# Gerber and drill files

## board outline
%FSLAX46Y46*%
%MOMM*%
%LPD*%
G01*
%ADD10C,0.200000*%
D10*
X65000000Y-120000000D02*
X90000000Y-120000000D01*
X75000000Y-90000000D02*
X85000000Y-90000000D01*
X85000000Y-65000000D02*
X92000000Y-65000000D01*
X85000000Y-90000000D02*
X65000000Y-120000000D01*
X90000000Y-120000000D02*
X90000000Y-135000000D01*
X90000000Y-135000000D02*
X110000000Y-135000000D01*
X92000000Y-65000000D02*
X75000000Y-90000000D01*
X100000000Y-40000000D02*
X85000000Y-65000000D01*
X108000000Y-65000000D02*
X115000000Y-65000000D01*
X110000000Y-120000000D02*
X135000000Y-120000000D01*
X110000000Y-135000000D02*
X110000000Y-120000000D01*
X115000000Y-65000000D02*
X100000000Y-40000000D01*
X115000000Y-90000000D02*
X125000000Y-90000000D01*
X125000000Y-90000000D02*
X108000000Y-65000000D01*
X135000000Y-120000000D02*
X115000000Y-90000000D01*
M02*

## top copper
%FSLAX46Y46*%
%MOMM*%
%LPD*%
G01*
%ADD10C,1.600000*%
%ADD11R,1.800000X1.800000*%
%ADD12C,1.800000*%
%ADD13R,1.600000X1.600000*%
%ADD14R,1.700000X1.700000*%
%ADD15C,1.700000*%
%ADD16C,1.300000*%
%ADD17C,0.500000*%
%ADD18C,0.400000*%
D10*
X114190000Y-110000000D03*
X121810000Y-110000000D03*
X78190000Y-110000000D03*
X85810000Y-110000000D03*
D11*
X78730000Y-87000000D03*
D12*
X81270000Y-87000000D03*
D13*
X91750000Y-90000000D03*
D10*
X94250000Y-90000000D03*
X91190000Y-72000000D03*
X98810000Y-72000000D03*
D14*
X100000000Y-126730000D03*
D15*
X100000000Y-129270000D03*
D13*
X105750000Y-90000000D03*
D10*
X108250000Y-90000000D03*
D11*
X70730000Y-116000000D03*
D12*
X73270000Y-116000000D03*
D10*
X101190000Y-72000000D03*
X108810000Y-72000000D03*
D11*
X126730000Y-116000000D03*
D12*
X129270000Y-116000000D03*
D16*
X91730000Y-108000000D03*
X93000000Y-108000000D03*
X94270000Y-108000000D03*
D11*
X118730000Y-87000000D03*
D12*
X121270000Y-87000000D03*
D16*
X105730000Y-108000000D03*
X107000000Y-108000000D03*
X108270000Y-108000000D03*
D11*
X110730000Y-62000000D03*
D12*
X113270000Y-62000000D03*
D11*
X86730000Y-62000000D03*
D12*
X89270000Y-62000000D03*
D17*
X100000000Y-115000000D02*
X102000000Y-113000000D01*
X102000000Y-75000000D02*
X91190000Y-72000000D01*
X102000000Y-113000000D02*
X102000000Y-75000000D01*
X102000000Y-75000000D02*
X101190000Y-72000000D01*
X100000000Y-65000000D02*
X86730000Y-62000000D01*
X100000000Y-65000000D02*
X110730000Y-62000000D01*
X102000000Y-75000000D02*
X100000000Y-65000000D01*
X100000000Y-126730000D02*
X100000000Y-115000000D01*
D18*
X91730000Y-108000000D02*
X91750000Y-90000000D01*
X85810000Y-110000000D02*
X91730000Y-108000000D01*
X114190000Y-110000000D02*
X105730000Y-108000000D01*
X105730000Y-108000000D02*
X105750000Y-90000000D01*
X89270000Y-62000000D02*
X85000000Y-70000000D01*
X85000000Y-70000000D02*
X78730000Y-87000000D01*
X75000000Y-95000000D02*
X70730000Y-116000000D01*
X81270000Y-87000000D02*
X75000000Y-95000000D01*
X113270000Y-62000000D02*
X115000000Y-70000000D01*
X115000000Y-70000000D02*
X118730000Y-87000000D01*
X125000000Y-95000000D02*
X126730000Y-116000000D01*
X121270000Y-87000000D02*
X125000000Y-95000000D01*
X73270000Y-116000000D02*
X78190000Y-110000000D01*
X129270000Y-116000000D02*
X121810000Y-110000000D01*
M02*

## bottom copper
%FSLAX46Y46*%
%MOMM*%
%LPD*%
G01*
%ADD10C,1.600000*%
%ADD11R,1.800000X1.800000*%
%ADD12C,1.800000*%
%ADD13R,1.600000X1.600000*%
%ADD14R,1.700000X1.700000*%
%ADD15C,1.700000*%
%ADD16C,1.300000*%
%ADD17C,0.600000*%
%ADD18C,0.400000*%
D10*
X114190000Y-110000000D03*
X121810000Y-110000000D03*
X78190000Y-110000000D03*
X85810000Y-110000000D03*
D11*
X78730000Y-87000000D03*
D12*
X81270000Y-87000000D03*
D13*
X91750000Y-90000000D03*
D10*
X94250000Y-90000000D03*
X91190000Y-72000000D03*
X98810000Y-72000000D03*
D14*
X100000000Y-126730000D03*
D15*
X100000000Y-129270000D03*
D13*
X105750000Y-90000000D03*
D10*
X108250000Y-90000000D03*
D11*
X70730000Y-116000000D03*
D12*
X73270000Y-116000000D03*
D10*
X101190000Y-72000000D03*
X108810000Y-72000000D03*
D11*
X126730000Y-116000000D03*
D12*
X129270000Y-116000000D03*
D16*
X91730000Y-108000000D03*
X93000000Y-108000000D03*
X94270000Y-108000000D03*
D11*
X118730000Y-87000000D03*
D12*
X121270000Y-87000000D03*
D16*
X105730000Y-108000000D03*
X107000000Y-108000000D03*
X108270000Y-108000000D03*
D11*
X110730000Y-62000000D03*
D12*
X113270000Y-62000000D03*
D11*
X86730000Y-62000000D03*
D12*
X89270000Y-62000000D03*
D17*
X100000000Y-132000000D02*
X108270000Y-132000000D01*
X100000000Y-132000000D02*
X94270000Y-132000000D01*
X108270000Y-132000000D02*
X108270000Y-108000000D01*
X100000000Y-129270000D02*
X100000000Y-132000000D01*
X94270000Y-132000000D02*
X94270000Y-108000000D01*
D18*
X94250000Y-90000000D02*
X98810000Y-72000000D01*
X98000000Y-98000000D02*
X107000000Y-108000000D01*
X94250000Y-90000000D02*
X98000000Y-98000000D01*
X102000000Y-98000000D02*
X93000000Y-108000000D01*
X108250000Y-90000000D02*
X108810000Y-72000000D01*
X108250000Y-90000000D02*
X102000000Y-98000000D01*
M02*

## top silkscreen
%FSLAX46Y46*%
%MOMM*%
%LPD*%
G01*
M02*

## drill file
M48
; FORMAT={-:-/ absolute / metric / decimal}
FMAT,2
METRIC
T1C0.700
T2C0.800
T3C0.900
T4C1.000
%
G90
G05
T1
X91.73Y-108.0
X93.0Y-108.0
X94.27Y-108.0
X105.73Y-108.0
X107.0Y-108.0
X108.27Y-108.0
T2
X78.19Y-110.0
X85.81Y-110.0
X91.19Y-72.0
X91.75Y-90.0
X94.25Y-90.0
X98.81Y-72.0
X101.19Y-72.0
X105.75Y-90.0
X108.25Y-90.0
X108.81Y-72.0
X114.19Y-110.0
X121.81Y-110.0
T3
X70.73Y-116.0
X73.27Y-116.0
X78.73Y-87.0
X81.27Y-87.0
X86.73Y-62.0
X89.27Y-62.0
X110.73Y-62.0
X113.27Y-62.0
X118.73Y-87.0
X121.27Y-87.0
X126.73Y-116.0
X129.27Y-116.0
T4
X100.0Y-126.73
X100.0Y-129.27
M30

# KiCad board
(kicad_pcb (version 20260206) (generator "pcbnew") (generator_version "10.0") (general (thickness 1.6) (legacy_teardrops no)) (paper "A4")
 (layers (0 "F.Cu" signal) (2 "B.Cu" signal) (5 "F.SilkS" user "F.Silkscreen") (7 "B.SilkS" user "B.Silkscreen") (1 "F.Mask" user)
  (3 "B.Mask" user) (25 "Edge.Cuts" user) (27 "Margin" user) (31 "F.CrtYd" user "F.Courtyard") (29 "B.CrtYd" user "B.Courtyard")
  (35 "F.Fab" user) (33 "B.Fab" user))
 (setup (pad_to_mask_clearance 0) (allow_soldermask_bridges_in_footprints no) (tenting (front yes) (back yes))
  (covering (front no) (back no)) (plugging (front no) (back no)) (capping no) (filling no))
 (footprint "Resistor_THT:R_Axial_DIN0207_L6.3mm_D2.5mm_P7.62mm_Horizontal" (layer "F.Cu") (at 118 110)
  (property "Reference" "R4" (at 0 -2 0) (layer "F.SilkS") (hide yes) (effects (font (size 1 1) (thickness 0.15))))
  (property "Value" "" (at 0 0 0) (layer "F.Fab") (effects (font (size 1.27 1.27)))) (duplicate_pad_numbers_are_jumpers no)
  (pad "1" thru_hole circle (at -3.81 0) (size 1.6 1.6) (drill 0.8) (layers "*.Cu" "*.Mask") (remove_unused_layers no) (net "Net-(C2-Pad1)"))
  (pad "2" thru_hole circle (at 3.81 0) (size 1.6 1.6) (drill 0.8) (layers "*.Cu" "*.Mask") (remove_unused_layers no) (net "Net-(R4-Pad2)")))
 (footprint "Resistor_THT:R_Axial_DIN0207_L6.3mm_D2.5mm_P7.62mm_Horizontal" (layer "F.Cu") (at 82 110)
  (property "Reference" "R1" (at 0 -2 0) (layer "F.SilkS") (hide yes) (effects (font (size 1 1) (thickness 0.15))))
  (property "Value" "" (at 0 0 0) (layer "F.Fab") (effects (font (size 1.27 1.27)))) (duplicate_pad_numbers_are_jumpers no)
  (pad "1" thru_hole circle (at -3.81 0) (size 1.6 1.6) (drill 0.8) (layers "*.Cu" "*.Mask") (remove_unused_layers no) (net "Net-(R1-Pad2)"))
  (pad "2" thru_hole circle (at 3.81 0) (size 1.6 1.6) (drill 0.8) (layers "*.Cu" "*.Mask") (remove_unused_layers no) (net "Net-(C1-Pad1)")))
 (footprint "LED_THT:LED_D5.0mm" (layer "F.Cu") (at 80 87)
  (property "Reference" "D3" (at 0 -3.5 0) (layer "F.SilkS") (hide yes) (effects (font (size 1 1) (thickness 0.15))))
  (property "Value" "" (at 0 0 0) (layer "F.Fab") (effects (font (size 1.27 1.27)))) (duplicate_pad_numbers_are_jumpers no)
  (pad "1" thru_hole rect (at -1.27 0) (size 1.8 1.8) (drill 0.9) (layers "*.Cu" "*.Mask") (remove_unused_layers no) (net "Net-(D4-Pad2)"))
  (pad "2" thru_hole circle (at 1.27 0) (size 1.8 1.8) (drill 0.9) (layers "*.Cu" "*.Mask") (remove_unused_layers no) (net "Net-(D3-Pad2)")))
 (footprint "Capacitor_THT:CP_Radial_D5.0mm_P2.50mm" (layer "F.Cu") (at 93 90)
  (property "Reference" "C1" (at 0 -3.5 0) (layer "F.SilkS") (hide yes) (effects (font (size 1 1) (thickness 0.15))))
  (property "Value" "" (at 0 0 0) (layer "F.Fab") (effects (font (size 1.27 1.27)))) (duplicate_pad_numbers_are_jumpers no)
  (pad "1" thru_hole rect (at -1.25 0) (size 1.6 1.6) (drill 0.8) (layers "*.Cu" "*.Mask") (remove_unused_layers no) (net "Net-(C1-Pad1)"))
  (pad "2" thru_hole circle (at 1.25 0) (size 1.6 1.6) (drill 0.8) (layers "*.Cu" "*.Mask") (remove_unused_layers no) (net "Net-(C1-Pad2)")))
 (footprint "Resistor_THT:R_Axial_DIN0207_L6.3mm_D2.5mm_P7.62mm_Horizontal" (layer "F.Cu") (at 95 72)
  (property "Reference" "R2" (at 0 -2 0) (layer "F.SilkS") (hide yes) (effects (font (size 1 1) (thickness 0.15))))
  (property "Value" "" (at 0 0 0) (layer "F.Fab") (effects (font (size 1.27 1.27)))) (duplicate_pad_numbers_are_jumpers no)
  (pad "1" thru_hole circle (at -3.81 0) (size 1.6 1.6) (drill 0.8) (layers "*.Cu" "*.Mask") (remove_unused_layers no) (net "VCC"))
  (pad "2" thru_hole circle (at 3.81 0) (size 1.6 1.6) (drill 0.8) (layers "*.Cu" "*.Mask") (remove_unused_layers no) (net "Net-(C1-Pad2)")))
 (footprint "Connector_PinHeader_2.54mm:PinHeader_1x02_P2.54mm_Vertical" (layer "F.Cu") (at 100 128)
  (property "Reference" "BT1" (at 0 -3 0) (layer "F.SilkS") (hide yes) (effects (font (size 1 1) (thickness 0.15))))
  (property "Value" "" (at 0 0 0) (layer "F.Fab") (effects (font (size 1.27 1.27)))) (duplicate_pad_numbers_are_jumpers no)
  (pad "1" thru_hole rect (at 0 -1.27) (size 1.7 1.7) (drill 1) (layers "*.Cu" "*.Mask") (remove_unused_layers no) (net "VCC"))
  (pad "2" thru_hole circle (at 0 1.27) (size 1.7 1.7) (drill 1) (layers "*.Cu" "*.Mask") (remove_unused_layers no) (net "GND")))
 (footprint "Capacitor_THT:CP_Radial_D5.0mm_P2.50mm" (layer "F.Cu") (at 107 90)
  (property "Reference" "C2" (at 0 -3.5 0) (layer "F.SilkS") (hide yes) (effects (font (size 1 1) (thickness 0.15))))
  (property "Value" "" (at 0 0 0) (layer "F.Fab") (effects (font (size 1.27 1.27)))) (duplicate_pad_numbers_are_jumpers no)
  (pad "1" thru_hole rect (at -1.25 0) (size 1.6 1.6) (drill 0.8) (layers "*.Cu" "*.Mask") (remove_unused_layers no) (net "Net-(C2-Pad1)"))
  (pad "2" thru_hole circle (at 1.25 0) (size 1.6 1.6) (drill 0.8) (layers "*.Cu" "*.Mask") (remove_unused_layers no) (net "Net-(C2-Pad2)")))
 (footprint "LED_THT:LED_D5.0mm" (layer "F.Cu") (at 72 116)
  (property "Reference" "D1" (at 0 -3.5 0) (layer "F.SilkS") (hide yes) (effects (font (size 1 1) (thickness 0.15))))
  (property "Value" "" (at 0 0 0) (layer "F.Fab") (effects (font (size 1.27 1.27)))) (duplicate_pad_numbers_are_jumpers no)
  (pad "1" thru_hole rect (at -1.27 0) (size 1.8 1.8) (drill 0.9) (layers "*.Cu" "*.Mask") (remove_unused_layers no) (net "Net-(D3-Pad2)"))
  (pad "2" thru_hole circle (at 1.27 0) (size 1.8 1.8) (drill 0.9) (layers "*.Cu" "*.Mask") (remove_unused_layers no) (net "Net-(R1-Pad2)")))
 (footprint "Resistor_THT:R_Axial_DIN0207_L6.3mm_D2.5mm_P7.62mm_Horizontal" (layer "F.Cu") (at 105 72)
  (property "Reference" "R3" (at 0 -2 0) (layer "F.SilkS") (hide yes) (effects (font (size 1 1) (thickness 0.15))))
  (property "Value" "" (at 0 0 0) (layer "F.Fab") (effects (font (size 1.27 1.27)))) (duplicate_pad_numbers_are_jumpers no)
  (pad "1" thru_hole circle (at -3.81 0) (size 1.6 1.6) (drill 0.8) (layers "*.Cu" "*.Mask") (remove_unused_layers no) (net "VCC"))
  (pad "2" thru_hole circle (at 3.81 0) (size 1.6 1.6) (drill 0.8) (layers "*.Cu" "*.Mask") (remove_unused_layers no) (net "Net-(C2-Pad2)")))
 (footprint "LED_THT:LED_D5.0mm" (layer "F.Cu") (at 128 116)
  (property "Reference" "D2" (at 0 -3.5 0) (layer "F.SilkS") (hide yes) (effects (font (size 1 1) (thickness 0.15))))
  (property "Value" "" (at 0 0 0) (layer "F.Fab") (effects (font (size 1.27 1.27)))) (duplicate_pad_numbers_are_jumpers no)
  (pad "1" thru_hole rect (at -1.27 0) (size 1.8 1.8) (drill 0.9) (layers "*.Cu" "*.Mask") (remove_unused_layers no) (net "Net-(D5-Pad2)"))
  (pad "2" thru_hole circle (at 1.27 0) (size 1.8 1.8) (drill 0.9) (layers "*.Cu" "*.Mask") (remove_unused_layers no) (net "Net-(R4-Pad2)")))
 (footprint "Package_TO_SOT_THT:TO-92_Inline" (layer "F.Cu") (at 93 108)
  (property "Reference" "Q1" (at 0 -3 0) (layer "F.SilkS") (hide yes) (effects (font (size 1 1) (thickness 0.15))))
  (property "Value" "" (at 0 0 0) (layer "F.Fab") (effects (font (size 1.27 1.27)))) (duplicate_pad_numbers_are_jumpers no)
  (pad "1" thru_hole circle (at -1.27 0) (size 1.3 1.3) (drill 0.7) (layers "*.Cu" "*.Mask") (remove_unused_layers no) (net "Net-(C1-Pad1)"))
  (pad "2" thru_hole circle (at 0 0) (size 1.3 1.3) (drill 0.7) (layers "*.Cu" "*.Mask") (remove_unused_layers no) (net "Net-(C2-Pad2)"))
  (pad "3" thru_hole circle (at 1.27 0) (size 1.3 1.3) (drill 0.7) (layers "*.Cu" "*.Mask") (remove_unused_layers no) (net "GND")))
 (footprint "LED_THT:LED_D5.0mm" (layer "F.Cu") (at 120 87)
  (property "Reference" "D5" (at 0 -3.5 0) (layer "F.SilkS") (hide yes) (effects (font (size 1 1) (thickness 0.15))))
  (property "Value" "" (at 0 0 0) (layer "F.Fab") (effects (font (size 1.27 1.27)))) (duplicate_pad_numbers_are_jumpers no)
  (pad "1" thru_hole rect (at -1.27 0) (size 1.8 1.8) (drill 0.9) (layers "*.Cu" "*.Mask") (remove_unused_layers no) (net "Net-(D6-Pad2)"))
  (pad "2" thru_hole circle (at 1.27 0) (size 1.8 1.8) (drill 0.9) (layers "*.Cu" "*.Mask") (remove_unused_layers no) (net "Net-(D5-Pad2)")))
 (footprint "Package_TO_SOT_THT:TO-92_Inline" (layer "F.Cu") (at 107 108)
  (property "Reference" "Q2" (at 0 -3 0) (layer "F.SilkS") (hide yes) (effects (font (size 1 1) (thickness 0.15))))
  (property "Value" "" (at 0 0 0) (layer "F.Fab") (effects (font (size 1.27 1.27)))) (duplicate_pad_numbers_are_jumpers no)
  (pad "1" thru_hole circle (at -1.27 0) (size 1.3 1.3) (drill 0.7) (layers "*.Cu" "*.Mask") (remove_unused_layers no) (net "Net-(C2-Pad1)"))
  (pad "2" thru_hole circle (at 0 0) (size 1.3 1.3) (drill 0.7) (layers "*.Cu" "*.Mask") (remove_unused_layers no) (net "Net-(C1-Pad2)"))
  (pad "3" thru_hole circle (at 1.27 0) (size 1.3 1.3) (drill 0.7) (layers "*.Cu" "*.Mask") (remove_unused_layers no) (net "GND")))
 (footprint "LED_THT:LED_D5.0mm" (layer "F.Cu") (at 112 62)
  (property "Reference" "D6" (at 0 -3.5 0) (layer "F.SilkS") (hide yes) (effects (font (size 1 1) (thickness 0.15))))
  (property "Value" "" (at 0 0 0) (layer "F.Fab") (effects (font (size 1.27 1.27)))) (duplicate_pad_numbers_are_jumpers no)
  (pad "1" thru_hole rect (at -1.27 0) (size 1.8 1.8) (drill 0.9) (layers "*.Cu" "*.Mask") (remove_unused_layers no) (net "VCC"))
  (pad "2" thru_hole circle (at 1.27 0) (size 1.8 1.8) (drill 0.9) (layers "*.Cu" "*.Mask") (remove_unused_layers no) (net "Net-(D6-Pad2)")))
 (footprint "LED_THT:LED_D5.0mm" (layer "F.Cu") (at 88 62)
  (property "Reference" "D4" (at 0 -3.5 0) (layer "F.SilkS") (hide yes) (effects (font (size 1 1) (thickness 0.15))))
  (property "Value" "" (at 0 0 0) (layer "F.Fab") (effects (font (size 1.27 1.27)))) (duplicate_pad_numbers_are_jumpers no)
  (pad "1" thru_hole rect (at -1.27 0) (size 1.8 1.8) (drill 0.9) (layers "*.Cu" "*.Mask") (remove_unused_layers no) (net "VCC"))
  (pad "2" thru_hole circle (at 1.27 0) (size 1.8 1.8) (drill 0.9) (layers "*.Cu" "*.Mask") (remove_unused_layers no) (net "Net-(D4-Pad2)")))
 (gr_line (start 65 120) (end 90 120) (stroke (width 0.2) (type solid)) (layer "Edge.Cuts"))
 (gr_line (start 75 90) (end 85 90) (stroke (width 0.2) (type solid)) (layer "Edge.Cuts"))
 (gr_line (start 85 65) (end 92 65) (stroke (width 0.2) (type solid)) (layer "Edge.Cuts"))
 (gr_line (start 85 90) (end 65 120) (stroke (width 0.2) (type solid)) (layer "Edge.Cuts"))
 (gr_line (start 90 120) (end 90 135) (stroke (width 0.2) (type solid)) (layer "Edge.Cuts"))
 (gr_line (start 90 135) (end 110 135) (stroke (width 0.2) (type solid)) (layer "Edge.Cuts"))
 (gr_line (start 92 65) (end 75 90) (stroke (width 0.2) (type solid)) (layer "Edge.Cuts"))
 (gr_line (start 100 40) (end 85 65) (stroke (width 0.2) (type solid)) (layer "Edge.Cuts"))
 (gr_line (start 108 65) (end 115 65) (stroke (width 0.2) (type solid)) (layer "Edge.Cuts"))
 (gr_line (start 110 120) (end 135 120) (stroke (width 0.2) (type solid)) (layer "Edge.Cuts"))
 (gr_line (start 110 135) (end 110 120) (stroke (width 0.2) (type solid)) (layer "Edge.Cuts"))
 (gr_line (start 115 65) (end 100 40) (stroke (width 0.2) (type solid)) (layer "Edge.Cuts"))
 (gr_line (start 115 90) (end 125 90) (stroke (width 0.2) (type solid)) (layer "Edge.Cuts"))
 (gr_line (start 125 90) (end 108 65) (stroke (width 0.2) (type solid)) (layer "Edge.Cuts"))
 (gr_line (start 135 120) (end 115 90) (stroke (width 0.2) (type solid)) (layer "Edge.Cuts"))
 (segment (start 100 115) (end 102 113) (width 0.5) (layer "F.Cu") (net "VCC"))
 (segment (start 102 75) (end 91.19 72) (width 0.5) (layer "F.Cu") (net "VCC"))
 (segment (start 102 113) (end 102 75) (width 0.5) (layer "F.Cu") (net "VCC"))
 (segment (start 102 75) (end 101.19 72) (width 0.5) (layer "F.Cu") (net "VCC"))
 (segment (start 100 65) (end 86.73 62) (width 0.5) (layer "F.Cu") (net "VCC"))
 (segment (start 100 65) (end 110.73 62) (width 0.5) (layer "F.Cu") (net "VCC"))
 (segment (start 102 75) (end 100 65) (width 0.5) (layer "F.Cu") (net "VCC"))
 (segment (start 100 126.73) (end 100 115) (width 0.5) (layer "F.Cu") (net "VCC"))
 (segment (start 100 132) (end 108.27 132) (width 0.6) (layer "B.Cu") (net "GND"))
 (segment (start 100 132) (end 94.27 132) (width 0.6) (layer "B.Cu") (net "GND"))
 (segment (start 108.27 132) (end 108.27 108) (width 0.6) (layer "B.Cu") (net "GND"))
 (segment (start 100 129.27) (end 100 132) (width 0.6) (layer "B.Cu") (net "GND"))
 (segment (start 94.27 132) (end 94.27 108) (width 0.6) (layer "B.Cu") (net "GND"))
 (segment (start 91.73 108) (end 91.75 90) (width 0.4) (layer "F.Cu") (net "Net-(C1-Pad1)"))
 (segment (start 85.81 110) (end 91.73 108) (width 0.4) (layer "F.Cu") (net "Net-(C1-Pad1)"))
 (segment (start 114.19 110) (end 105.73 108) (width 0.4) (layer "F.Cu") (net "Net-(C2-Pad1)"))
 (segment (start 105.73 108) (end 105.75 90) (width 0.4) (layer "F.Cu") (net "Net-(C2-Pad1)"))
 (segment (start 94.25 90) (end 98.81 72) (width 0.4) (layer "B.Cu") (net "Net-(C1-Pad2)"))
 (segment (start 98 98) (end 107 108) (width 0.4) (layer "B.Cu") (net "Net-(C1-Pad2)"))
 (segment (start 94.25 90) (end 98 98) (width 0.4) (layer "B.Cu") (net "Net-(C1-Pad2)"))
 (segment (start 102 98) (end 93 108) (width 0.4) (layer "B.Cu") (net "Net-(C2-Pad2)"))
 (segment (start 108.25 90) (end 108.81 72) (width 0.4) (layer "B.Cu") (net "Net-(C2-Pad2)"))
 (segment (start 108.25 90) (end 102 98) (width 0.4) (layer "B.Cu") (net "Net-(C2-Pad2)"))
 (segment (start 89.27 62) (end 85 70) (width 0.4) (layer "F.Cu") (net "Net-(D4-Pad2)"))
 (segment (start 85 70) (end 78.73 87) (width 0.4) (layer "F.Cu") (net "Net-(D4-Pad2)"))
 (segment (start 75 95) (end 70.73 116) (width 0.4) (layer "F.Cu") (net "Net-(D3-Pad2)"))
 (segment (start 81.27 87) (end 75 95) (width 0.4) (layer "F.Cu") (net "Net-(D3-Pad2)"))
 (segment (start 113.27 62) (end 115 70) (width 0.4) (layer "F.Cu") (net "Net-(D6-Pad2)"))
 (segment (start 115 70) (end 118.73 87) (width 0.4) (layer "F.Cu") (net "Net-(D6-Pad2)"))
 (segment (start 125 95) (end 126.73 116) (width 0.4) (layer "F.Cu") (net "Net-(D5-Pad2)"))
 (segment (start 121.27 87) (end 125 95) (width 0.4) (layer "F.Cu") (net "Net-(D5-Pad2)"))
 (segment (start 73.27 116) (end 78.19 110) (width 0.4) (layer "F.Cu") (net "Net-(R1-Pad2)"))
 (segment (start 129.27 116) (end 121.81 110) (width 0.4) (layer "F.Cu") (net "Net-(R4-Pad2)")))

